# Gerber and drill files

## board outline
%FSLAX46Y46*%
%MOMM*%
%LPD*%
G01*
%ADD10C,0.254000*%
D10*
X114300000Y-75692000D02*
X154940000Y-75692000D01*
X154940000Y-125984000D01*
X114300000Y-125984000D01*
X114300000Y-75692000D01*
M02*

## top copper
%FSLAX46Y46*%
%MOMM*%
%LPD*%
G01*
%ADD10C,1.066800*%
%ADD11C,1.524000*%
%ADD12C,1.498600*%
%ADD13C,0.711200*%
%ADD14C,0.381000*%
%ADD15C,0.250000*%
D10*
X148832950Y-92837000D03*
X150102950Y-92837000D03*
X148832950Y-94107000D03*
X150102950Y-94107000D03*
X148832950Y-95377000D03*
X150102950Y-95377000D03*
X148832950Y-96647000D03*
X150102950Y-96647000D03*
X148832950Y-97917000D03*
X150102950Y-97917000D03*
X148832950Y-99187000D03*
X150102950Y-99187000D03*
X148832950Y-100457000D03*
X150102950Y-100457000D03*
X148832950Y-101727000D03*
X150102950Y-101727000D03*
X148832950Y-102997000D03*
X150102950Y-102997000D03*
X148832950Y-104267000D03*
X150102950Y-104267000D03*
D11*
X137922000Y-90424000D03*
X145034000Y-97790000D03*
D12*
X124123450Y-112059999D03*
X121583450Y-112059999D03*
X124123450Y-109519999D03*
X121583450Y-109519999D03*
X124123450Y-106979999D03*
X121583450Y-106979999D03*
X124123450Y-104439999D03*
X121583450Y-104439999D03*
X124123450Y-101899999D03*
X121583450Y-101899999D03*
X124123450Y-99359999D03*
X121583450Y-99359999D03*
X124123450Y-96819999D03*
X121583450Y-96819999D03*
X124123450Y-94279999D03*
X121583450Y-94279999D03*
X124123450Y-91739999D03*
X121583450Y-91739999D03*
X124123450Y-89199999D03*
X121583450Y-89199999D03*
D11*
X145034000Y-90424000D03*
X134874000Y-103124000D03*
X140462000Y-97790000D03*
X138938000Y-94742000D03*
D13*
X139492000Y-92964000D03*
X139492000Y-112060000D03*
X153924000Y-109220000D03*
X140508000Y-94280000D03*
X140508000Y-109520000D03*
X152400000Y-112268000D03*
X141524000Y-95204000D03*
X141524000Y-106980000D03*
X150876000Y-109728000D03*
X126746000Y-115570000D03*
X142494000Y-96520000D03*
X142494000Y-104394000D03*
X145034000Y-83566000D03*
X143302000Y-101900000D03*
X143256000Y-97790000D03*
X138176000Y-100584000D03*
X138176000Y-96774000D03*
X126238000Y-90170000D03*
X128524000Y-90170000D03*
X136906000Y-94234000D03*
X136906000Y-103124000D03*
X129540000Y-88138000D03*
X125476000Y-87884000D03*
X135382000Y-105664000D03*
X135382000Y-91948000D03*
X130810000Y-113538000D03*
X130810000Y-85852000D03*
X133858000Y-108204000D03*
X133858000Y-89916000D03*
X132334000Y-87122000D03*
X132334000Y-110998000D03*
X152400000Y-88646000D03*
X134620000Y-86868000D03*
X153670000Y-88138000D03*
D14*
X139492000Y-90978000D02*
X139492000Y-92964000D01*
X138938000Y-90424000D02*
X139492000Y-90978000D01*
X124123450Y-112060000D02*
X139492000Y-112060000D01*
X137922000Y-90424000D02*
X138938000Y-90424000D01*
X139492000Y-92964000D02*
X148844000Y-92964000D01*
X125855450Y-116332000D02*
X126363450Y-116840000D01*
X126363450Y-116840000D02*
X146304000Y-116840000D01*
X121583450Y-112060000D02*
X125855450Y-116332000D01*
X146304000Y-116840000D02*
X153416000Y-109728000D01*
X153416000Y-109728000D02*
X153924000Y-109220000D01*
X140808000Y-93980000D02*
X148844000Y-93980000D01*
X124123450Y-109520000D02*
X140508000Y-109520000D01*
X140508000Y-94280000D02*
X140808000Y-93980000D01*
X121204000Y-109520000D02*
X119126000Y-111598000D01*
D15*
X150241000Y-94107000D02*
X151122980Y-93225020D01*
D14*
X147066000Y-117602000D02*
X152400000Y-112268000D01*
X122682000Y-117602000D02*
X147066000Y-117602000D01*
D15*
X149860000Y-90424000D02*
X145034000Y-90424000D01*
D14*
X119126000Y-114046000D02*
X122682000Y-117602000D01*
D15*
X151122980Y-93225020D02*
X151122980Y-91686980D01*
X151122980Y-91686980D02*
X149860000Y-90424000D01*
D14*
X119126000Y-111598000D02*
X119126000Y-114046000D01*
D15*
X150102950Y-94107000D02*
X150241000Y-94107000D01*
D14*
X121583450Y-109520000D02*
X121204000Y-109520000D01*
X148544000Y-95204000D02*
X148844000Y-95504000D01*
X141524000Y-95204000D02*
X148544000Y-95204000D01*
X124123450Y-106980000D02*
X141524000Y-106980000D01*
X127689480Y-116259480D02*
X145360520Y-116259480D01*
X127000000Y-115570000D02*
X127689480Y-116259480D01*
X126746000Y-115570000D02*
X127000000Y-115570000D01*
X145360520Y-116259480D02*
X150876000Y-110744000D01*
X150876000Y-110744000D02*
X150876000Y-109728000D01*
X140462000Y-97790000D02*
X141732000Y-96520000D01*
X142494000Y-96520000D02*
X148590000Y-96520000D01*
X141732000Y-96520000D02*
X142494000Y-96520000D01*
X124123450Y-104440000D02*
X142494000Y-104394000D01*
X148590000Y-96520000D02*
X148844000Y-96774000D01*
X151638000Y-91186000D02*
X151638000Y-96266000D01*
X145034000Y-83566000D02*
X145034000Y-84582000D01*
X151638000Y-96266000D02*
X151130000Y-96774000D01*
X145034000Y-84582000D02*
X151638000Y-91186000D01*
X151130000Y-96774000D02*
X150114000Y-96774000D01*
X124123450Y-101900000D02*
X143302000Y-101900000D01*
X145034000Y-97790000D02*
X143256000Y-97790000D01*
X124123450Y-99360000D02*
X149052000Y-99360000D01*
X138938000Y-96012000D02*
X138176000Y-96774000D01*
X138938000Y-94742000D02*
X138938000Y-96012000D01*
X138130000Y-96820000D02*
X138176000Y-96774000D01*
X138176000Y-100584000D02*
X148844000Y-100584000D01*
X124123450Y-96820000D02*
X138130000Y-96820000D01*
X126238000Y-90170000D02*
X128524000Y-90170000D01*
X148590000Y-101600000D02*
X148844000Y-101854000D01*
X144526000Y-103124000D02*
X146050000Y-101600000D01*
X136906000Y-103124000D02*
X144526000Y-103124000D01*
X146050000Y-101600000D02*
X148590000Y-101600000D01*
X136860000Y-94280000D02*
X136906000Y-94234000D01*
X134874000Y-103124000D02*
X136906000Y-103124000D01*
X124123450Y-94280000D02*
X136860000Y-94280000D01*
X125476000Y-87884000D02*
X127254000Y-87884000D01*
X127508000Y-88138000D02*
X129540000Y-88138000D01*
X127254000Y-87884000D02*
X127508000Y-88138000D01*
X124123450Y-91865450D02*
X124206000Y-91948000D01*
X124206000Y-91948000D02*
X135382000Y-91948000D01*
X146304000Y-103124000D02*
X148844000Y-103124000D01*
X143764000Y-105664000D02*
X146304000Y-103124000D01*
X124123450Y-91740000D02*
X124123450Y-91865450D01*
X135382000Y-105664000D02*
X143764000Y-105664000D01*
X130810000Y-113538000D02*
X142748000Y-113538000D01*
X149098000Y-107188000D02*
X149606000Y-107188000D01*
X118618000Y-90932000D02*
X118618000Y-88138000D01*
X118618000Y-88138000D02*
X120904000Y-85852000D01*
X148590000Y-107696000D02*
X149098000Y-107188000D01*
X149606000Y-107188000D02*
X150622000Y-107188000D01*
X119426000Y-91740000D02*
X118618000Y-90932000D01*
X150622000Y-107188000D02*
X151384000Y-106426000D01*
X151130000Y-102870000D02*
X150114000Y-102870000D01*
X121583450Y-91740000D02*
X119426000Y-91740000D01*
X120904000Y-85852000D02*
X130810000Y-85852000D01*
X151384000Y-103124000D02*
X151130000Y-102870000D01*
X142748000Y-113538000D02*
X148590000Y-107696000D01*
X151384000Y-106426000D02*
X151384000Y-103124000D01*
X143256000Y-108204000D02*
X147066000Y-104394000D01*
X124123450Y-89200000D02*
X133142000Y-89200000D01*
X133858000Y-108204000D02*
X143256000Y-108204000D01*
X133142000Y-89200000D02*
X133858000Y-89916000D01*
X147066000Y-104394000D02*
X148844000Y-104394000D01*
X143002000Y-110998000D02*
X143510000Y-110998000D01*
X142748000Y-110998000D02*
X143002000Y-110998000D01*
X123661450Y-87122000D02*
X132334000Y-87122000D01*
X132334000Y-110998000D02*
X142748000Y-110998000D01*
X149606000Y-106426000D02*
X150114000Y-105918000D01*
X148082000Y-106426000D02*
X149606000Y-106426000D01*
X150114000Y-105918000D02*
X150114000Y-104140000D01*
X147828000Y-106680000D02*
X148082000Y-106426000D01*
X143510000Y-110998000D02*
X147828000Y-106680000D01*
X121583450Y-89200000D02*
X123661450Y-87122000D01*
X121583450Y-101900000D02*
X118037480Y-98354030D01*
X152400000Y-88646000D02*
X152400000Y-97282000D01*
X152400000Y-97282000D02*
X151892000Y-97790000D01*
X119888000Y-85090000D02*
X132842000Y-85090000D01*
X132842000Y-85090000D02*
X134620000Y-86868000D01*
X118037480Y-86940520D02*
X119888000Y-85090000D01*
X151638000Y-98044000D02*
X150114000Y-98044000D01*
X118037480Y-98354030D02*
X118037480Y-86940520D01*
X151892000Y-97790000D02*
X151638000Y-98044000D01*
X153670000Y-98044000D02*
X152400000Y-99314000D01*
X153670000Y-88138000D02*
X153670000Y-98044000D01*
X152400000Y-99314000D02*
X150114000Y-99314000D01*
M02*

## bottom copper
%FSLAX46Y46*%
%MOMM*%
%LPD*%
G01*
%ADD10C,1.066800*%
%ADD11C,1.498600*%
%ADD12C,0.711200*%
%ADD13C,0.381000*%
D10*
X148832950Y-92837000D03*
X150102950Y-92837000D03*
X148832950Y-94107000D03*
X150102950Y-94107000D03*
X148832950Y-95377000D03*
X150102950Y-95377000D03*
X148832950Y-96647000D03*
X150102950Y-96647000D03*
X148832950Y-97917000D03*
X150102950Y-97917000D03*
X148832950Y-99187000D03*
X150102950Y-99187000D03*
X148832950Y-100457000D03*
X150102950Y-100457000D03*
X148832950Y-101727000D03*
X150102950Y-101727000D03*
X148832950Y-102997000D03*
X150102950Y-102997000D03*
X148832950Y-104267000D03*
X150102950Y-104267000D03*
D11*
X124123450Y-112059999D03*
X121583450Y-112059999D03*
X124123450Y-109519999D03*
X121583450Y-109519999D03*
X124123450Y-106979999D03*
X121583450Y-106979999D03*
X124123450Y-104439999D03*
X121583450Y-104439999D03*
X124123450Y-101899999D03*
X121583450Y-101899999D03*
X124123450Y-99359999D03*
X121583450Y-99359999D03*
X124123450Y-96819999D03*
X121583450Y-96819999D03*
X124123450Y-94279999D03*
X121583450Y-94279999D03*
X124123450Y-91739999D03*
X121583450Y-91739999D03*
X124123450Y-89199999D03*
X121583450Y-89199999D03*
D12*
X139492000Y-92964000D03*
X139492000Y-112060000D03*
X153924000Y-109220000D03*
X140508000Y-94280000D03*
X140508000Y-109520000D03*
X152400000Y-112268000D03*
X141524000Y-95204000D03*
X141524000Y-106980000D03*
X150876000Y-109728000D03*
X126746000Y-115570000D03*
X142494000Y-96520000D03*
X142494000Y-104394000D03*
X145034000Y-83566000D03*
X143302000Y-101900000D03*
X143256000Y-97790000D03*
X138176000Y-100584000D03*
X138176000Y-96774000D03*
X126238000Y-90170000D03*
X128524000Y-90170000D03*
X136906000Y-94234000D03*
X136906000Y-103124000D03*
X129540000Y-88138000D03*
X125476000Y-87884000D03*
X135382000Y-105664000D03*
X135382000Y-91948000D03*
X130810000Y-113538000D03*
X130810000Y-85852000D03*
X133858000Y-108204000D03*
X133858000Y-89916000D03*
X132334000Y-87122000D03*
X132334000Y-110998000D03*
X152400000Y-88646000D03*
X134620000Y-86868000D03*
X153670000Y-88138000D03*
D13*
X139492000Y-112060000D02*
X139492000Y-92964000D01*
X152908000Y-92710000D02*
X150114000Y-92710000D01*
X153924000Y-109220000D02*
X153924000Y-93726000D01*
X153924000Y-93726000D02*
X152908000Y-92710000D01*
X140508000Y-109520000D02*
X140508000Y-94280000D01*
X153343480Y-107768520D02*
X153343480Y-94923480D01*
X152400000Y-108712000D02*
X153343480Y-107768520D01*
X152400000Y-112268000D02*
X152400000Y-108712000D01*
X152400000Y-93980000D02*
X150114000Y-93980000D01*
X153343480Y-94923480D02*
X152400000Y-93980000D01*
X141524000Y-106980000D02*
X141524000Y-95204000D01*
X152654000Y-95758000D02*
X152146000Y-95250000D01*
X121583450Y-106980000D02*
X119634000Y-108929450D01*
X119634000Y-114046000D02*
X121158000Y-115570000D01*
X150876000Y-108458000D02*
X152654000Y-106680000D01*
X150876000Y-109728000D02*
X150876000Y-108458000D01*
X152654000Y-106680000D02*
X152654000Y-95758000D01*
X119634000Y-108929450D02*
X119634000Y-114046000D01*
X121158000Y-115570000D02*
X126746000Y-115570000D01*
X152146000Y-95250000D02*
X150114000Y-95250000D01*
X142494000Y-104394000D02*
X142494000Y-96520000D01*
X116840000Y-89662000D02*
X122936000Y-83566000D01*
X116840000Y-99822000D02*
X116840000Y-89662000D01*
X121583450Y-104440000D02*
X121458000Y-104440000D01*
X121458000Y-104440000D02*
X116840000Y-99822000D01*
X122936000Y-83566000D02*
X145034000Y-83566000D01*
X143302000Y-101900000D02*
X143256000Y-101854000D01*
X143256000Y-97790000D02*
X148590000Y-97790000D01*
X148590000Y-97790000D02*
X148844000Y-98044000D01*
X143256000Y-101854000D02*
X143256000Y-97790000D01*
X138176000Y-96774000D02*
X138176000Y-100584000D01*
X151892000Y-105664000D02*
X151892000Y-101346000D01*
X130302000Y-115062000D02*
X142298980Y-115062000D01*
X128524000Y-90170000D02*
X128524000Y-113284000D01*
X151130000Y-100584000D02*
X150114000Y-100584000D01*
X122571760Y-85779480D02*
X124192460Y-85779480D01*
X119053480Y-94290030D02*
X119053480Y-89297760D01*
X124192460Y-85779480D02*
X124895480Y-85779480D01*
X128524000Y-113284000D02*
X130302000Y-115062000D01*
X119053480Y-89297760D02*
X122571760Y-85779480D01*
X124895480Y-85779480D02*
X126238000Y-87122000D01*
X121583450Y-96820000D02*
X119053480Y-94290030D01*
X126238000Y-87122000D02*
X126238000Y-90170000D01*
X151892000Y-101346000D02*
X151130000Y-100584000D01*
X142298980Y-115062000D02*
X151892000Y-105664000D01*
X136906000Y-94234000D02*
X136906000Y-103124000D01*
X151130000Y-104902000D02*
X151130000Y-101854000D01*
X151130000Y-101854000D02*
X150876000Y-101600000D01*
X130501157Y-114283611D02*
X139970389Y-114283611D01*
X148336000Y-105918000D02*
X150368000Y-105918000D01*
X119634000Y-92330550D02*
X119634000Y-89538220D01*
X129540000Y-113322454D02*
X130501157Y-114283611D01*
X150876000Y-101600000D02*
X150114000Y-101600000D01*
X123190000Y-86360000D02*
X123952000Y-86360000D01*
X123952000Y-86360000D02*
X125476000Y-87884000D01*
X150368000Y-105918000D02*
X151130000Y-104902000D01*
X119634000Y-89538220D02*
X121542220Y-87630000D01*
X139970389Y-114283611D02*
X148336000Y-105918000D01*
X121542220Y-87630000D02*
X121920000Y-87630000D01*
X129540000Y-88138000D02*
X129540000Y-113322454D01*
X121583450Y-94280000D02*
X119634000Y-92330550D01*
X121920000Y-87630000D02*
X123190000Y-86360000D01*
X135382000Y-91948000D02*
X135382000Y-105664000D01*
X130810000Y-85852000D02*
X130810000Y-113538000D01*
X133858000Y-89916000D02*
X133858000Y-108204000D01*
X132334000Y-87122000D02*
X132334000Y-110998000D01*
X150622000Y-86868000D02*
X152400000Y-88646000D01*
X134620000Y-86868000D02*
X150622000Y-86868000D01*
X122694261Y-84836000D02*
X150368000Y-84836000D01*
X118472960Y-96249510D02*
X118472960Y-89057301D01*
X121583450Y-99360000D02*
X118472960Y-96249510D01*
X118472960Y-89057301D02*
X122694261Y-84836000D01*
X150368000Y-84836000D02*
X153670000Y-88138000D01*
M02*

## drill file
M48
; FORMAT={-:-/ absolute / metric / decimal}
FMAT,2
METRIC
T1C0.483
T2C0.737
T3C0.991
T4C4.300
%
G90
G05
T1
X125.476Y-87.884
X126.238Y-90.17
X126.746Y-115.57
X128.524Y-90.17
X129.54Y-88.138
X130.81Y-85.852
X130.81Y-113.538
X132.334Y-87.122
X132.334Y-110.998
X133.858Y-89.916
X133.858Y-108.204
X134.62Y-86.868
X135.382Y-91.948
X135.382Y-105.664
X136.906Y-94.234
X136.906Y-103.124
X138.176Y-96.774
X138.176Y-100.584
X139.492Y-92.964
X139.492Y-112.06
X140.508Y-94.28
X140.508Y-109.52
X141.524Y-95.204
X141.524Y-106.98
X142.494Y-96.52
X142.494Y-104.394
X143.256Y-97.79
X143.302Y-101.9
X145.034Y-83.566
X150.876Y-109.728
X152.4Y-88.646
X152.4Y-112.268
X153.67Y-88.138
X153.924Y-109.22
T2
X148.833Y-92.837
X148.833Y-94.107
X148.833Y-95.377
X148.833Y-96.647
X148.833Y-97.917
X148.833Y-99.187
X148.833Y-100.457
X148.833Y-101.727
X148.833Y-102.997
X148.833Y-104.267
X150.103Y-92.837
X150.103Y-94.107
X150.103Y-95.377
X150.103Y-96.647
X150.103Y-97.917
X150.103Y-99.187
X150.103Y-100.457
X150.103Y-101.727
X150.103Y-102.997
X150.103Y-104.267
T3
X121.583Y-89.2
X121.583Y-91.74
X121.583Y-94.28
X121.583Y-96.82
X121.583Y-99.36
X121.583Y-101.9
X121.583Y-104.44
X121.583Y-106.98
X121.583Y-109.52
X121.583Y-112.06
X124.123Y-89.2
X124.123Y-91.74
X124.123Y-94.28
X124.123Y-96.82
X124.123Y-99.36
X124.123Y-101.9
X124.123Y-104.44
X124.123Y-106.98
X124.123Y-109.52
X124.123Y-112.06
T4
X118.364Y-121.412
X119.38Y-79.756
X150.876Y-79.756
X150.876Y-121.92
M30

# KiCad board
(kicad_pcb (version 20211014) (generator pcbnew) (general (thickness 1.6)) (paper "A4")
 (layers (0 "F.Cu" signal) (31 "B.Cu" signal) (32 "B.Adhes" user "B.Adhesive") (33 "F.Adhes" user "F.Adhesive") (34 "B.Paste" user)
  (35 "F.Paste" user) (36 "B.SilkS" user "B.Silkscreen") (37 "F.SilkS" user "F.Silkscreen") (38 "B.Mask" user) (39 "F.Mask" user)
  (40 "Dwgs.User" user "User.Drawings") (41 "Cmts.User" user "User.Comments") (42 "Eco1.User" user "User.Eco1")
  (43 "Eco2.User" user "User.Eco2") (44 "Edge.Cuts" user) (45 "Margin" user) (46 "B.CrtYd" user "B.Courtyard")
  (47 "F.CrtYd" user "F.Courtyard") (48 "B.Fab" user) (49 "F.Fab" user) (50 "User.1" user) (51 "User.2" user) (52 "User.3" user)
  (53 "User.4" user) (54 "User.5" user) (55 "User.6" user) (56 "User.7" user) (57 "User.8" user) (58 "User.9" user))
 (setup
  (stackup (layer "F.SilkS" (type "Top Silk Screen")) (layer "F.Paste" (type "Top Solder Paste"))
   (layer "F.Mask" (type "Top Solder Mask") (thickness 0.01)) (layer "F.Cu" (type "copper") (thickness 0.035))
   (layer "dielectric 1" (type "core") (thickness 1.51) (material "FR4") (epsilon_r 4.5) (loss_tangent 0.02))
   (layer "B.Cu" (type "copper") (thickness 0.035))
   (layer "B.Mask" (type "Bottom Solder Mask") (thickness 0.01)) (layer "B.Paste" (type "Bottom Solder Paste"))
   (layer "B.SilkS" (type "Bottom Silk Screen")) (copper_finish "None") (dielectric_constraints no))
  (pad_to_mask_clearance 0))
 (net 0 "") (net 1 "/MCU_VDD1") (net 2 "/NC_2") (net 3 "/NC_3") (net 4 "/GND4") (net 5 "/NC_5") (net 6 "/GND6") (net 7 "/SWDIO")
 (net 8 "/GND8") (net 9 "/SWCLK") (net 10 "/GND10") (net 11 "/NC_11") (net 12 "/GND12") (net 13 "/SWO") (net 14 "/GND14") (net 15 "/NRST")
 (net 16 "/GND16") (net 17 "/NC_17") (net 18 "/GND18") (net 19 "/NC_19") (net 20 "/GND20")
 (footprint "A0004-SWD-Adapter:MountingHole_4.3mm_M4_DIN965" (layer "F.Cu") (at 150.876 79.756)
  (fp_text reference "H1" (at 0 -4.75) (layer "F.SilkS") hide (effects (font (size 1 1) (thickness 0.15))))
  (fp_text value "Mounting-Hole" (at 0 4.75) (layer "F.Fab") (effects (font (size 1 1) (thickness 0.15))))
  (pad "" np_thru_hole circle (at 0 0) (size 4.3 4.3) (drill 4.3) (layers *.Cu *.Mask)))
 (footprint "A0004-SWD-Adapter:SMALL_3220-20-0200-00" (layer "F.Cu") (at 150.10295 98.552 -90)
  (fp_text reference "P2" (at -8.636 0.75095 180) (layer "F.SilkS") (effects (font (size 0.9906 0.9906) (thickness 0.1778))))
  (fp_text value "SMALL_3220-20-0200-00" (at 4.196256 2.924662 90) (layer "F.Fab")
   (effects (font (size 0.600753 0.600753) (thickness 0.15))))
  (pad "1" thru_hole circle (at -5.715 1.27 270) (size 1.0668 1.0668) (drill 0.7366) (layers *.Cu *.Mask) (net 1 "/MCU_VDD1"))
  (pad "2" thru_hole circle (at -5.715 0 270) (size 1.0668 1.0668) (drill 0.7366) (layers *.Cu *.Mask) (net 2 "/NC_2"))
  (pad "3" thru_hole circle (at -4.445 1.27 270) (size 1.0668 1.0668) (drill 0.7366) (layers *.Cu *.Mask) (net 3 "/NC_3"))
  (pad "4" thru_hole circle (at -4.445 0 270) (size 1.0668 1.0668) (drill 0.7366) (layers *.Cu *.Mask) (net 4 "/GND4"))
  (pad "5" thru_hole circle (at -3.175 1.27 270) (size 1.0668 1.0668) (drill 0.7366) (layers *.Cu *.Mask) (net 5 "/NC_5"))
  (pad "6" thru_hole circle (at -3.175 0 270) (size 1.0668 1.0668) (drill 0.7366) (layers *.Cu *.Mask) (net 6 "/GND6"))
  (pad "7" thru_hole circle (at -1.905 1.27 270) (size 1.0668 1.0668) (drill 0.7366) (layers *.Cu *.Mask) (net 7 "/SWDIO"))
  (pad "8" thru_hole circle (at -1.905 0 270) (size 1.0668 1.0668) (drill 0.7366) (layers *.Cu *.Mask) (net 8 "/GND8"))
  (pad "9" thru_hole circle (at -0.635 1.27 270) (size 1.0668 1.0668) (drill 0.7366) (layers *.Cu *.Mask) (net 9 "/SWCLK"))
  (pad "10" thru_hole circle (at -0.635 0 270) (size 1.0668 1.0668) (drill 0.7366) (layers *.Cu *.Mask) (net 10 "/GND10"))
  (pad "11" thru_hole circle (at 0.635 1.27 270) (size 1.0668 1.0668) (drill 0.7366) (layers *.Cu *.Mask) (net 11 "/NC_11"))
  (pad "12" thru_hole circle (at 0.635 0 270) (size 1.0668 1.0668) (drill 0.7366) (layers *.Cu *.Mask) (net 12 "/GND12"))
  (pad "13" thru_hole circle (at 1.905 1.27 270) (size 1.0668 1.0668) (drill 0.7366) (layers *.Cu *.Mask) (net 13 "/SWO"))
  (pad "14" thru_hole circle (at 1.905 0 270) (size 1.0668 1.0668) (drill 0.7366) (layers *.Cu *.Mask) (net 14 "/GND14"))
  (pad "15" thru_hole circle (at 3.175 1.27 270) (size 1.0668 1.0668) (drill 0.7366) (layers *.Cu *.Mask) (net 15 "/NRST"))
  (pad "16" thru_hole circle (at 3.175 0 270) (size 1.0668 1.0668) (drill 0.7366) (layers *.Cu *.Mask) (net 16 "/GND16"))
  (pad "17" thru_hole circle (at 4.445 1.27 270) (size 1.0668 1.0668) (drill 0.7366) (layers *.Cu *.Mask) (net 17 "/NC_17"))
  (pad "18" thru_hole circle (at 4.445 0 270) (size 1.0668 1.0668) (drill 0.7366) (layers *.Cu *.Mask) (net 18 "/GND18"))
  (pad "19" thru_hole circle (at 5.715 1.27 270) (size 1.0668 1.0668) (drill 0.7366) (layers *.Cu *.Mask) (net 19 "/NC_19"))
  (pad "20" thru_hole circle (at 5.715 0 270) (size 1.0668 1.0668) (drill 0.7366) (layers *.Cu *.Mask) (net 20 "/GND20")))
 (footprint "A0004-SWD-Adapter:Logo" (layer "F.Cu") (at 135.382 119.888)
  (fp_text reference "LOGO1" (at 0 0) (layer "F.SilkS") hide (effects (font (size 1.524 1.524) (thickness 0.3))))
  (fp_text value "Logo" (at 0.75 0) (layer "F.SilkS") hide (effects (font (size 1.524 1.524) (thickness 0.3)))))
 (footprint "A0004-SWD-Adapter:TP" (layer "F.Cu") (at 137.922 90.424)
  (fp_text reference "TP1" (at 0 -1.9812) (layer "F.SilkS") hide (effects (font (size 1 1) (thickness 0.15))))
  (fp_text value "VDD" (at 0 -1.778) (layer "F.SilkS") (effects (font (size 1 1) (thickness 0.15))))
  (pad "1" smd circle (at 0 0) (size 1.524 1.524) (layers "F.Cu" "F.Paste" "F.Mask") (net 1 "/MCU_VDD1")))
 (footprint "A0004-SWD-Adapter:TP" (layer "F.Cu") (at 145.034 97.79)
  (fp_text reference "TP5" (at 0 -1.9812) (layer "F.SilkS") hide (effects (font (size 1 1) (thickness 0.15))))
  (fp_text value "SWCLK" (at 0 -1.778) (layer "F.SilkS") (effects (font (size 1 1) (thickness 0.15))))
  (pad "1" smd circle (at 0 0) (size 1.524 1.524) (layers "F.Cu" "F.Paste" "F.Mask") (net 9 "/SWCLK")))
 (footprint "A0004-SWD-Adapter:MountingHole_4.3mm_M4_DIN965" (layer "F.Cu") (at 118.364 121.412)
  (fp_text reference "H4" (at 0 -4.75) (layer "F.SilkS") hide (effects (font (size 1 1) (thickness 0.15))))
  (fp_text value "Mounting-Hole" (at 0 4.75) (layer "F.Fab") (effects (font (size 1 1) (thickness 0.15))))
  (pad "" np_thru_hole circle (at 0 0) (size 4.3 4.3) (drill 4.3) (layers *.Cu *.Mask)))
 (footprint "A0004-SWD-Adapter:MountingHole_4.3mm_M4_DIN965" (layer "F.Cu") (at 119.38 79.756)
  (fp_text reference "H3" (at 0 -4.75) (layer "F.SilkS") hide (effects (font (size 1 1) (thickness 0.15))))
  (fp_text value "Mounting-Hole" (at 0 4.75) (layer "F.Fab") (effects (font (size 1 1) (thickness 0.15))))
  (pad "" np_thru_hole circle (at 0 0) (size 4.3 4.3) (drill 4.3) (layers *.Cu *.Mask)))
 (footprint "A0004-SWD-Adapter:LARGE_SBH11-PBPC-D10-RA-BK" (layer "F.Cu") (at 121.58345 112.059999 90)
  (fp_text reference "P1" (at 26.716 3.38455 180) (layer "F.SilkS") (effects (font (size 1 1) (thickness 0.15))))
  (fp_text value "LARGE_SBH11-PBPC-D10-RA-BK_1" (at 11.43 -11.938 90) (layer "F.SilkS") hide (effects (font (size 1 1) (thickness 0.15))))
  (pad "1" thru_hole circle (at 0 2.54 90) (size 1.4986 1.4986) (drill 0.9906) (layers *.Cu *.Mask) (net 1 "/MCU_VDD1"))
  (pad "2" thru_hole circle (at 0 0 90) (size 1.4986 1.4986) (drill 0.9906) (layers *.Cu *.Mask) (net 2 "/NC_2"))
  (pad "3" thru_hole circle (at 2.54 2.54 90) (size 1.4986 1.4986) (drill 0.9906) (layers *.Cu *.Mask) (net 3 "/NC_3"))
  (pad "4" thru_hole circle (at 2.54 0 90) (size 1.4986 1.4986) (drill 0.9906) (layers *.Cu *.Mask) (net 4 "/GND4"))
  (pad "5" thru_hole circle (at 5.08 2.54 90) (size 1.4986 1.4986) (drill 0.9906) (layers *.Cu *.Mask) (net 5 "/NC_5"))
  (pad "6" thru_hole circle (at 5.08 0 90) (size 1.4986 1.4986) (drill 0.9906) (layers *.Cu *.Mask) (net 6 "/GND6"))
  (pad "7" thru_hole circle (at 7.62 2.54 90) (size 1.4986 1.4986) (drill 0.9906) (layers *.Cu *.Mask) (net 7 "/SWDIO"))
  (pad "8" thru_hole circle (at 7.62 0 90) (size 1.4986 1.4986) (drill 0.9906) (layers *.Cu *.Mask) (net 8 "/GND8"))
  (pad "9" thru_hole circle (at 10.16 2.54 90) (size 1.4986 1.4986) (drill 0.9906) (layers *.Cu *.Mask) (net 9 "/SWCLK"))
  (pad "10" thru_hole circle (at 10.16 0 90) (size 1.4986 1.4986) (drill 0.9906) (layers *.Cu *.Mask) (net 10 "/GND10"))
  (pad "11" thru_hole circle (at 12.7 2.54 90) (size 1.4986 1.4986) (drill 0.9906) (layers *.Cu *.Mask) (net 11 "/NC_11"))
  (pad "12" thru_hole circle (at 12.7 0 90) (size 1.4986 1.4986) (drill 0.9906) (layers *.Cu *.Mask) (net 12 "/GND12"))
  (pad "13" thru_hole circle (at 15.24 2.54 90) (size 1.4986 1.4986) (drill 0.9906) (layers *.Cu *.Mask) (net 13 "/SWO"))
  (pad "14" thru_hole circle (at 15.24 0 90) (size 1.4986 1.4986) (drill 0.9906) (layers *.Cu *.Mask) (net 14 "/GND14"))
  (pad "15" thru_hole circle (at 17.78 2.54 90) (size 1.4986 1.4986) (drill 0.9906) (layers *.Cu *.Mask) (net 15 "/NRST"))
  (pad "16" thru_hole circle (at 17.78 0 90) (size 1.4986 1.4986) (drill 0.9906) (layers *.Cu *.Mask) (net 16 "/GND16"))
  (pad "17" thru_hole circle (at 20.32 2.54 90) (size 1.4986 1.4986) (drill 0.9906) (layers *.Cu *.Mask) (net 17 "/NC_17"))
  (pad "18" thru_hole circle (at 20.32 0 90) (size 1.4986 1.4986) (drill 0.9906) (layers *.Cu *.Mask) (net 18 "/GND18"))
  (pad "19" thru_hole circle (at 22.86 2.54 90) (size 1.4986 1.4986) (drill 0.9906) (layers *.Cu *.Mask) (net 19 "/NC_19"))
  (pad "20" thru_hole circle (at 22.86 0 90) (size 1.4986 1.4986) (drill 0.9906) (layers *.Cu *.Mask) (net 20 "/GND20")))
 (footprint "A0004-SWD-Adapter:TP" (layer "F.Cu") (at 145.034 90.424)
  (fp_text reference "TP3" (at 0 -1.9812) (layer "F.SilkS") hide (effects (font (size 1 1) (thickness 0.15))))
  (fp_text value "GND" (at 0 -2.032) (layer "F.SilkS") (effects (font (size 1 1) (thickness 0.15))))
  (pad "1" smd circle (at 0 0) (size 1.524 1.524) (layers "F.Cu" "F.Paste" "F.Mask") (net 4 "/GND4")))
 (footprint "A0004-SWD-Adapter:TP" (layer "F.Cu") (at 134.874 103.124)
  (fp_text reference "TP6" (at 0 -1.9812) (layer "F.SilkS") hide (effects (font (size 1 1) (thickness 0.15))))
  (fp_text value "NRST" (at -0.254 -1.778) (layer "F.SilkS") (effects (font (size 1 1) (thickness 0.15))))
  (pad "1" smd circle (at 0 0) (size 1.524 1.524) (layers "F.Cu" "F.Paste" "F.Mask") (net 15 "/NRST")))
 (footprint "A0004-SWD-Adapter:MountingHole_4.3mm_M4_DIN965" (layer "F.Cu") (at 150.876 121.92)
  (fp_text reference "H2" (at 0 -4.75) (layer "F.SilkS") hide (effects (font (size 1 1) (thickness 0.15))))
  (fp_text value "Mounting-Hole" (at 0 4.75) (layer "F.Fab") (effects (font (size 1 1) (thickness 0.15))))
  (pad "" np_thru_hole circle (at 0 0) (size 4.3 4.3) (drill 4.3) (layers *.Cu *.Mask)))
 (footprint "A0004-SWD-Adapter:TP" (layer "F.Cu") (at 140.462 97.79)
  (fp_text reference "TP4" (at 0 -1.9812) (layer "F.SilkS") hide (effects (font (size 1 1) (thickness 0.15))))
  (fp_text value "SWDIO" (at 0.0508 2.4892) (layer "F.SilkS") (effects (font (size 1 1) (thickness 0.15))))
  (pad "1" smd circle (at 0 0) (size 1.524 1.524) (layers "F.Cu" "F.Paste" "F.Mask") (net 7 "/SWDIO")))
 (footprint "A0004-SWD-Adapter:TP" (layer "F.Cu") (at 138.938 94.742)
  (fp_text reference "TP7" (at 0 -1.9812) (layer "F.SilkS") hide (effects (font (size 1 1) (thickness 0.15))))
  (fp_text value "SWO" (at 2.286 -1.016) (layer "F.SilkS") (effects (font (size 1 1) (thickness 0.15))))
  (pad "1" smd circle (at 0 0) (size 1.524 1.524) (layers "F.Cu" "F.Paste" "F.Mask") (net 13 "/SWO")))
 (gr_rect (start 114.3 75.692) (end 154.94 125.984) (layer "Edge.Cuts") (width 0.254) (fill none))
 (segment (start 139.492 90.978) (end 139.492 92.964) (width 0.381) (layer "F.Cu") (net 1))
 (segment (start 138.938 90.424) (end 139.492 90.978) (width 0.381) (layer "F.Cu") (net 1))
 (segment (start 124.12345 112.06) (end 139.492 112.06) (width 0.381) (layer "F.Cu") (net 1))
 (segment (start 137.922 90.424) (end 138.938 90.424) (width 0.381) (layer "F.Cu") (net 1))
 (segment (start 139.492 92.964) (end 148.844 92.964) (width 0.381) (layer "F.Cu") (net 1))
 (via (at 139.492 92.964) (size 0.7112) (drill 0.4826) (layers "F.Cu" "B.Cu") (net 1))
 (via (at 139.492 112.06) (size 0.7112) (drill 0.4826) (layers "F.Cu" "B.Cu") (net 1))
 (segment (start 139.492 112.06) (end 139.492 92.964) (width 0.381) (layer "B.Cu") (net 1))
 (segment (start 125.85545 116.332) (end 126.36345 116.84) (width 0.381) (layer "F.Cu") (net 2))
 (segment (start 126.36345 116.84) (end 146.304 116.84) (width 0.381) (layer "F.Cu") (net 2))
 (segment (start 121.58345 112.06) (end 125.85545 116.332) (width 0.381) (layer "F.Cu") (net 2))
 (segment (start 146.304 116.84) (end 153.416 109.728) (width 0.381) (layer "F.Cu") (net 2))
 (segment (start 153.416 109.728) (end 153.924 109.22) (width 0.381) (layer "F.Cu") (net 2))
 (via (at 153.924 109.22) (size 0.7112) (drill 0.4826) (layers "F.Cu" "B.Cu") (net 2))
 (segment (start 152.908 92.71) (end 150.114 92.71) (width 0.381) (layer "B.Cu") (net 2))
 (segment (start 153.924 109.22) (end 153.924 93.726) (width 0.381) (layer "B.Cu") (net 2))
 (segment (start 153.924 93.726) (end 152.908 92.71) (width 0.381) (layer "B.Cu") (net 2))
 (segment (start 140.808 93.98) (end 148.844 93.98) (width 0.381) (layer "F.Cu") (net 3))
 (segment (start 124.12345 109.52) (end 140.508 109.52) (width 0.381) (layer "F.Cu") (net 3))
 (segment (start 140.508 94.28) (end 140.808 93.98) (width 0.381) (layer "F.Cu") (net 3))
 (via (at 140.508 94.28) (size 0.7112) (drill 0.4826) (layers "F.Cu" "B.Cu") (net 3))
 (via (at 140.508 109.52) (size 0.7112) (drill 0.4826) (layers "F.Cu" "B.Cu") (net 3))
 (segment (start 140.508 109.52) (end 140.508 94.28) (width 0.381) (layer "B.Cu") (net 3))
 (segment (start 121.204 109.52) (end 119.126 111.598) (width 0.381) (layer "F.Cu") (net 4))
 (segment (start 150.241 94.107) (end 151.12298 93.22502) (width 0.25) (layer "F.Cu") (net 4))
 (segment (start 147.066 117.602) (end 152.4 112.268) (width 0.381) (layer "F.Cu") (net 4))
 (segment (start 122.682 117.602) (end 147.066 117.602) (width 0.381) (layer "F.Cu") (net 4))
 (segment (start 149.86 90.424) (end 145.034 90.424) (width 0.25) (layer "F.Cu") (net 4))
 (segment (start 119.126 114.046) (end 122.682 117.602) (width 0.381) (layer "F.Cu") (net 4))
 (segment (start 151.12298 93.22502) (end 151.12298 91.68698) (width 0.25) (layer "F.Cu") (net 4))
 (segment (start 151.12298 91.68698) (end 149.86 90.424) (width 0.25) (layer "F.Cu") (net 4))
 (segment (start 119.126 111.598) (end 119.126 114.046) (width 0.381) (layer "F.Cu") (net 4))
 (segment (start 150.10295 94.107) (end 150.241 94.107) (width 0.25) (layer "F.Cu") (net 4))
 (segment (start 121.58345 109.52) (end 121.204 109.52) (width 0.381) (layer "F.Cu") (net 4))
 (via (at 152.4 112.268) (size 0.7112) (drill 0.4826) (layers "F.Cu" "B.Cu") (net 4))
 (segment (start 153.34348 107.76852) (end 153.34348 94.92348) (width 0.381) (layer "B.Cu") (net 4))
 (segment (start 152.4 108.712) (end 153.34348 107.76852) (width 0.381) (layer "B.Cu") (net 4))
 (segment (start 152.4 112.268) (end 152.4 108.712) (width 0.381) (layer "B.Cu") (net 4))
 (segment (start 152.4 93.98) (end 150.114 93.98) (width 0.381) (layer "B.Cu") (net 4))
 (segment (start 153.34348 94.92348) (end 152.4 93.98) (width 0.381) (layer "B.Cu") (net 4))
 (segment (start 148.544 95.204) (end 148.844 95.504) (width 0.381) (layer "F.Cu") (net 5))
 (segment (start 141.524 95.204) (end 148.544 95.204) (width 0.381) (layer "F.Cu") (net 5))
 (segment (start 124.12345 106.98) (end 141.524 106.98) (width 0.381) (layer "F.Cu") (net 5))
 (via (at 141.524 95.204) (size 0.7112) (drill 0.4826) (layers "F.Cu" "B.Cu") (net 5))
 (via (at 141.524 106.98) (size 0.7112) (drill 0.4826) (layers "F.Cu" "B.Cu") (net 5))
 (segment (start 141.524 106.98) (end 141.524 95.204) (width 0.381) (layer "B.Cu") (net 5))
 (segment (start 127.68948 116.25948) (end 145.36052 116.25948) (width 0.381) (layer "F.Cu") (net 6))
 (segment (start 127 115.57) (end 127.68948 116.25948) (width 0.381) (layer "F.Cu") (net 6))
 (segment (start 126.746 115.57) (end 127 115.57) (width 0.381) (layer "F.Cu") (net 6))
 (segment (start 145.36052 116.25948) (end 150.876 110.744) (width 0.381) (layer "F.Cu") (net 6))
 (segment (start 150.876 110.744) (end 150.876 109.728) (width 0.381) (layer "F.Cu") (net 6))
 (via (at 150.876 109.728) (size 0.7112) (drill 0.4826) (layers "F.Cu" "B.Cu") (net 6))
 (via (at 126.746 115.57) (size 0.7112) (drill 0.4826) (layers "F.Cu" "B.Cu") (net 6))
 (segment (start 152.654 95.758) (end 152.146 95.25) (width 0.381) (layer "B.Cu") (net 6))
 (segment (start 121.58345 106.98) (end 119.634 108.92945) (width 0.381) (layer "B.Cu") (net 6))
 (segment (start 119.634 114.046) (end 121.158 115.57) (width 0.381) (layer "B.Cu") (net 6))
 (segment (start 150.876 108.458) (end 152.654 106.68) (width 0.381) (layer "B.Cu") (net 6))
 (segment (start 150.876 109.728) (end 150.876 108.458) (width 0.381) (layer "B.Cu") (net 6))
 (segment (start 152.654 106.68) (end 152.654 95.758) (width 0.381) (layer "B.Cu") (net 6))
 (segment (start 119.634 108.92945) (end 119.634 114.046) (width 0.381) (layer "B.Cu") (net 6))
 (segment (start 121.158 115.57) (end 126.746 115.57) (width 0.381) (layer "B.Cu") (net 6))
 (segment (start 152.146 95.25) (end 150.114 95.25) (width 0.381) (layer "B.Cu") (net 6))
 (segment (start 140.462 97.79) (end 141.732 96.52) (width 0.381) (layer "F.Cu") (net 7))
 (segment (start 142.494 96.52) (end 148.59 96.52) (width 0.381) (layer "F.Cu") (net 7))
 (segment (start 141.732 96.52) (end 142.494 96.52) (width 0.381) (layer "F.Cu") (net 7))
 (segment (start 124.12345 104.44) (end 142.494 104.394) (width 0.381) (layer "F.Cu") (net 7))
 (segment (start 148.59 96.52) (end 148.844 96.774) (width 0.381) (layer "F.Cu") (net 7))
 (via (at 142.494 96.52) (size 0.7112) (drill 0.4826) (layers "F.Cu" "B.Cu") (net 7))
 (via (at 142.494 104.394) (size 0.7112) (drill 0.4826) (layers "F.Cu" "B.Cu") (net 7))
 (segment (start 142.494 104.394) (end 142.494 96.52) (width 0.381) (layer "B.Cu") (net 7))
 (segment (start 151.638 91.186) (end 151.638 96.266) (width 0.381) (layer "F.Cu") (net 8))
 (segment (start 145.034 83.566) (end 145.034 84.582) (width 0.381) (layer "F.Cu") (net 8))
 (segment (start 151.638 96.266) (end 151.13 96.774) (width 0.381) (layer "F.Cu") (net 8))
 (segment (start 145.034 84.582) (end 151.638 91.186) (width 0.381) (layer "F.Cu") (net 8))
 (segment (start 151.13 96.774) (end 150.114 96.774) (width 0.381) (layer "F.Cu") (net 8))
 (via (at 145.034 83.566) (size 0.7112) (drill 0.4826) (layers "F.Cu" "B.Cu") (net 8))
 (segment (start 116.84 89.662) (end 122.936 83.566) (width 0.381) (layer "B.Cu") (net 8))
 (segment (start 116.84 99.822) (end 116.84 89.662) (width 0.381) (layer "B.Cu") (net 8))
 (segment (start 121.58345 104.44) (end 121.458 104.44) (width 0.381) (layer "B.Cu") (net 8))
 (segment (start 121.458 104.44) (end 116.84 99.822) (width 0.381) (layer "B.Cu") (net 8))
 (segment (start 122.936 83.566) (end 145.034 83.566) (width 0.381) (layer "B.Cu") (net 8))
 (segment (start 124.12345 101.9) (end 143.302 101.9) (width 0.381) (layer "F.Cu") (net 9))
 (segment (start 145.034 97.79) (end 143.256 97.79) (width 0.381) (layer "F.Cu") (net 9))
 (via (at 143.302 101.9) (size 0.7112) (drill 0.4826) (layers "F.Cu" "B.Cu") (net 9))
 (via (at 143.256 97.79) (size 0.7112) (drill 0.4826) (layers "F.Cu" "B.Cu") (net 9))
 (segment (start 143.302 101.9) (end 143.256 101.854) (width 0.381) (layer "B.Cu") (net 9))
 (segment (start 143.256 97.79) (end 148.59 97.79) (width 0.381) (layer "B.Cu") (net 9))
 (segment (start 148.59 97.79) (end 148.844 98.044) (width 0.381) (layer "B.Cu") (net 9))
 (segment (start 143.256 101.854) (end 143.256 97.79) (width 0.381) (layer "B.Cu") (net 9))
 (segment (start 124.12345 99.36) (end 149.052 99.36) (width 0.381) (layer "F.Cu") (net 11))
 (segment (start 138.938 96.012) (end 138.176 96.774) (width 0.381) (layer "F.Cu") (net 13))
 (segment (start 138.938 94.742) (end 138.938 96.012) (width 0.381) (layer "F.Cu") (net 13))
 (segment (start 138.13 96.82) (end 138.176 96.774) (width 0.381) (layer "F.Cu") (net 13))
 (segment (start 138.176 100.584) (end 148.844 100.584) (width 0.381) (layer "F.Cu") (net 13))
 (segment (start 124.12345 96.82) (end 138.13 96.82) (width 0.381) (layer "F.Cu") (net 13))
 (via (at 138.176 100.584) (size 0.7112) (drill 0.4826) (layers "F.Cu" "B.Cu") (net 13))
 (via (at 138.176 96.774) (size 0.7112) (drill 0.4826) (layers "F.Cu" "B.Cu") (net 13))
 (segment (start 138.176 96.774) (end 138.176 100.584) (width 0.381) (layer "B.Cu") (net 13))
 (segment (start 126.238 90.17) (end 128.524 90.17) (width 0.381) (layer "F.Cu") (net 14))
 (via (at 126.238 90.17) (size 0.7112) (drill 0.4826) (layers "F.Cu" "B.Cu") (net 14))
 (via (at 128.524 90.17) (size 0.7112) (drill 0.4826) (layers "F.Cu" "B.Cu") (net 14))
 (segment (start 151.892 105.664) (end 151.892 101.346) (width 0.381) (layer "B.Cu") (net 14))
 (segment (start 130.302 115.062) (end 142.29898 115.062) (width 0.381) (layer "B.Cu") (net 14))
 (segment (start 128.524 90.17) (end 128.524 113.284) (width 0.381) (layer "B.Cu") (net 14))
 (segment (start 151.13 100.584) (end 150.114 100.584) (width 0.381) (layer "B.Cu") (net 14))
 (segment (start 122.57176 85.77948) (end 124.19246 85.77948) (width 0.381) (layer "B.Cu") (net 14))
 (segment (start 119.05348 94.29003) (end 119.05348 89.29776) (width 0.381) (layer "B.Cu") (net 14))
 (segment (start 124.19246 85.77948) (end 124.89548 85.77948) (width 0.381) (layer "B.Cu") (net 14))
 (segment (start 128.524 113.284) (end 130.302 115.062) (width 0.381) (layer "B.Cu") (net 14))
 (segment (start 119.05348 89.29776) (end 122.57176 85.77948) (width 0.381) (layer "B.Cu") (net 14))
 (segment (start 124.89548 85.77948) (end 126.238 87.122) (width 0.381) (layer "B.Cu") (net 14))
 (segment (start 121.58345 96.82) (end 119.05348 94.29003) (width 0.381) (layer "B.Cu") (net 14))
 (segment (start 126.238 87.122) (end 126.238 90.17) (width 0.381) (layer "B.Cu") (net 14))
 (segment (start 151.892 101.346) (end 151.13 100.584) (width 0.381) (layer "B.Cu") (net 14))
 (segment (start 142.29898 115.062) (end 151.892 105.664) (width 0.381) (layer "B.Cu") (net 14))
 (segment (start 148.59 101.6) (end 148.844 101.854) (width 0.381) (layer "F.Cu") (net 15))
 (segment (start 144.526 103.124) (end 146.05 101.6) (width 0.381) (layer "F.Cu") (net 15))
 (segment (start 136.906 103.124) (end 144.526 103.124) (width 0.381) (layer "F.Cu") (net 15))
 (segment (start 146.05 101.6) (end 148.59 101.6) (width 0.381) (layer "F.Cu") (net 15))
 (segment (start 136.86 94.28) (end 136.906 94.234) (width 0.381) (layer "F.Cu") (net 15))
 (segment (start 134.874 103.124) (end 136.906 103.124) (width 0.381) (layer "F.Cu") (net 15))
 (segment (start 124.12345 94.28) (end 136.86 94.28) (width 0.381) (layer "F.Cu") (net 15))
 (via (at 136.906 94.234) (size 0.7112) (drill 0.4826) (layers "F.Cu" "B.Cu") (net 15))
 (via (at 136.906 103.124) (size 0.7112) (drill 0.4826) (layers "F.Cu" "B.Cu") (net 15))
 (segment (start 136.906 94.234) (end 136.906 103.124) (width 0.381) (layer "B.Cu") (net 15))
 (segment (start 125.476 87.884) (end 127.254 87.884) (width 0.381) (layer "F.Cu") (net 16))
 (segment (start 127.508 88.138) (end 129.54 88.138) (width 0.381) (layer "F.Cu") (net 16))
 (segment (start 127.254 87.884) (end 127.508 88.138) (width 0.381) (layer "F.Cu") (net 16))
 (via (at 129.54 88.138) (size 0.7112) (drill 0.4826) (layers "F.Cu" "B.Cu") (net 16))
 (via (at 125.476 87.884) (size 0.7112) (drill 0.4826) (layers "F.Cu" "B.Cu") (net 16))
 (segment (start 151.13 104.902) (end 151.13 101.854) (width 0.381) (layer "B.Cu") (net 16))
 (segment (start 151.13 101.854) (end 150.876 101.6) (width 0.381) (layer "B.Cu") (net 16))
 (segment (start 130.501157 114.283611) (end 139.970389 114.283611) (width 0.381) (layer "B.Cu") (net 16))
 (segment (start 148.336 105.918) (end 150.368 105.918) (width 0.381) (layer "B.Cu") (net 16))
 (segment (start 119.634 92.33055) (end 119.634 89.53822) (width 0.381) (layer "B.Cu") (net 16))
 (segment (start 129.54 113.322454) (end 130.501157 114.283611) (width 0.381) (layer "B.Cu") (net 16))
 (segment (start 150.876 101.6) (end 150.114 101.6) (width 0.381) (layer "B.Cu") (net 16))
 (segment (start 123.19 86.36) (end 123.952 86.36) (width 0.381) (layer "B.Cu") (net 16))
 (segment (start 123.952 86.36) (end 125.476 87.884) (width 0.381) (layer "B.Cu") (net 16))
 (segment (start 150.368 105.918) (end 151.13 104.902) (width 0.381) (layer "B.Cu") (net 16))
 (segment (start 119.634 89.53822) (end 121.54222 87.63) (width 0.381) (layer "B.Cu") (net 16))
 (segment (start 139.970389 114.283611) (end 148.336 105.918) (width 0.381) (layer "B.Cu") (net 16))
 (segment (start 121.54222 87.63) (end 121.92 87.63) (width 0.381) (layer "B.Cu") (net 16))
 (segment (start 129.54 88.138) (end 129.54 113.322454) (width 0.381) (layer "B.Cu") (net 16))
 (segment (start 121.58345 94.28) (end 119.634 92.33055) (width 0.381) (layer "B.Cu") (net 16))
 (segment (start 121.92 87.63) (end 123.19 86.36) (width 0.381) (layer "B.Cu") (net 16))
 (segment (start 124.12345 91.86545) (end 124.206 91.948) (width 0.381) (layer "F.Cu") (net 17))
 (segment (start 124.206 91.948) (end 135.382 91.948) (width 0.381) (layer "F.Cu") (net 17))
 (segment (start 146.304 103.124) (end 148.844 103.124) (width 0.381) (layer "F.Cu") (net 17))
 (segment (start 143.764 105.664) (end 146.304 103.124) (width 0.381) (layer "F.Cu") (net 17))
 (segment (start 124.12345 91.74) (end 124.12345 91.86545) (width 0.381) (layer "F.Cu") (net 17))
 (segment (start 135.382 105.664) (end 143.764 105.664) (width 0.381) (layer "F.Cu") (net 17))
 (via (at 135.382 105.664) (size 0.7112) (drill 0.4826) (layers "F.Cu" "B.Cu") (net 17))
 (via (at 135.382 91.948) (size 0.7112) (drill 0.4826) (layers "F.Cu" "B.Cu") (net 17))
 (segment (start 135.382 91.948) (end 135.382 105.664) (width 0.381) (layer "B.Cu") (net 17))
 (segment (start 130.81 113.538) (end 142.748 113.538) (width 0.381) (layer "F.Cu") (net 18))
 (segment (start 149.098 107.188) (end 149.606 107.188) (width 0.381) (layer "F.Cu") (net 18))
 (segment (start 118.618 90.932) (end 118.618 88.138) (width 0.381) (layer "F.Cu") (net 18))
 (segment (start 118.618 88.138) (end 120.904 85.852) (width 0.381) (layer "F.Cu") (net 18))
 (segment (start 148.59 107.696) (end 149.098 107.188) (width 0.381) (layer "F.Cu") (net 18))
 (segment (start 149.606 107.188) (end 150.622 107.188) (width 0.381) (layer "F.Cu") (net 18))
 (segment (start 119.426 91.74) (end 118.618 90.932) (width 0.381) (layer "F.Cu") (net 18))
 (segment (start 150.622 107.188) (end 151.384 106.426) (width 0.381) (layer "F.Cu") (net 18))
 (segment (start 151.13 102.87) (end 150.114 102.87) (width 0.381) (layer "F.Cu") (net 18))
 (segment (start 121.58345 91.74) (end 119.426 91.74) (width 0.381) (layer "F.Cu") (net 18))
 (segment (start 120.904 85.852) (end 130.81 85.852) (width 0.381) (layer "F.Cu") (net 18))
 (segment (start 151.384 103.124) (end 151.13 102.87) (width 0.381) (layer "F.Cu") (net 18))
 (segment (start 142.748 113.538) (end 148.59 107.696) (width 0.381) (layer "F.Cu") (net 18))
 (segment (start 151.384 106.426) (end 151.384 103.124) (width 0.381) (layer "F.Cu") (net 18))
 (via (at 130.81 113.538) (size 0.7112) (drill 0.4826) (layers "F.Cu" "B.Cu") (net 18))
 (via (at 130.81 85.852) (size 0.7112) (drill 0.4826) (layers "F.Cu" "B.Cu") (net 18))
 (segment (start 130.81 85.852) (end 130.81 113.538) (width 0.381) (layer "B.Cu") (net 18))
 (segment (start 143.256 108.204) (end 147.066 104.394) (width 0.381) (layer "F.Cu") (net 19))
 (segment (start 124.12345 89.2) (end 133.142 89.2) (width 0.381) (layer "F.Cu") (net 19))
 (segment (start 133.858 108.204) (end 143.256 108.204) (width 0.381) (layer "F.Cu") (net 19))
 (segment (start 133.142 89.2) (end 133.858 89.916) (width 0.381) (layer "F.Cu") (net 19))
 (segment (start 147.066 104.394) (end 148.844 104.394) (width 0.381) (layer "F.Cu") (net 19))
 (via (at 133.858 108.204) (size 0.7112) (drill 0.4826) (layers "F.Cu" "B.Cu") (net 19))
 (via (at 133.858 89.916) (size 0.7112) (drill 0.4826) (layers "F.Cu" "B.Cu") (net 19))
 (segment (start 133.858 89.916) (end 133.858 108.204) (width 0.381) (layer "B.Cu") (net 19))
 (segment (start 143.002 110.998) (end 143.51 110.998) (width 0.381) (layer "F.Cu") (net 20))
 (segment (start 142.748 110.998) (end 143.002 110.998) (width 0.381) (layer "F.Cu") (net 20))
 (segment (start 123.66145 87.122) (end 132.334 87.122) (width 0.381) (layer "F.Cu") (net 20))
 (segment (start 132.334 110.998) (end 142.748 110.998) (width 0.381) (layer "F.Cu") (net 20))
 (segment (start 149.606 106.426) (end 150.114 105.918) (width 0.381) (layer "F.Cu") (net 20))
 (segment (start 148.082 106.426) (end 149.606 106.426) (width 0.381) (layer "F.Cu") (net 20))
 (segment (start 150.114 105.918) (end 150.114 104.14) (width 0.381) (layer "F.Cu") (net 20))
 (segment (start 147.828 106.68) (end 148.082 106.426) (width 0.381) (layer "F.Cu") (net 20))
 (segment (start 143.51 110.998) (end 147.828 106.68) (width 0.381) (layer "F.Cu") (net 20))
 (segment (start 121.58345 89.2) (end 123.66145 87.122) (width 0.381) (layer "F.Cu") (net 20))
 (via (at 132.334 87.122) (size 0.7112) (drill 0.4826) (layers "F.Cu" "B.Cu") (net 20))
 (via (at 132.334 110.998) (size 0.7112) (drill 0.4826) (layers "F.Cu" "B.Cu") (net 20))
 (segment (start 132.334 87.122) (end 132.334 110.998) (width 0.381) (layer "B.Cu") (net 20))
 (segment (start 121.58345 101.9) (end 118.03748 98.35403) (width 0.381) (layer "F.Cu") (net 10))
 (segment (start 152.4 88.646) (end 152.4 97.282) (width 0.381) (layer "F.Cu") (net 10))
 (segment (start 152.4 97.282) (end 151.892 97.79) (width 0.381) (layer "F.Cu") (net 10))
 (segment (start 119.888 85.09) (end 132.842 85.09) (width 0.381) (layer "F.Cu") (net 10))
 (segment (start 132.842 85.09) (end 134.62 86.868) (width 0.381) (layer "F.Cu") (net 10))
 (segment (start 118.03748 86.94052) (end 119.888 85.09) (width 0.381) (layer "F.Cu") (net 10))
 (segment (start 151.638 98.044) (end 150.114 98.044) (width 0.381) (layer "F.Cu") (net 10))
 (segment (start 118.03748 98.35403) (end 118.03748 86.94052) (width 0.381) (layer "F.Cu") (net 10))
 (segment (start 151.892 97.79) (end 151.638 98.044) (width 0.381) (layer "F.Cu") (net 10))
 (via (at 152.4 88.646) (size 0.7112) (drill 0.4826) (layers "F.Cu" "B.Cu") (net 10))
 (via (at 134.62 86.868) (size 0.7112) (drill 0.4826) (layers "F.Cu" "B.Cu") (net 10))
 (segment (start 150.622 86.868) (end 152.4 88.646) (width 0.381) (layer "B.Cu") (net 10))
 (segment (start 134.62 86.868) (end 150.622 86.868) (width 0.381) (layer "B.Cu") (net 10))
 (segment (start 153.67 98.044) (end 152.4 99.314) (width 0.381) (layer "F.Cu") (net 12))
 (segment (start 153.67 88.138) (end 153.67 98.044) (width 0.381) (layer "F.Cu") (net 12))
 (segment (start 152.4 99.314) (end 150.114 99.314) (width 0.381) (layer "F.Cu") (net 12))
 (via (at 153.67 88.138) (size 0.7112) (drill 0.4826) (layers "F.Cu" "B.Cu") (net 12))
 (segment (start 122.694261 84.836) (end 150.368 84.836) (width 0.381) (layer "B.Cu") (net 12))
 (segment (start 118.47296 96.24951) (end 118.47296 89.057301) (width 0.381) (layer "B.Cu") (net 12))
 (segment (start 121.58345 99.36) (end 118.47296 96.24951) (width 0.381) (layer "B.Cu") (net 12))
 (segment (start 118.47296 89.057301) (end 122.694261 84.836) (width 0.381) (layer "B.Cu") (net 12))
 (segment (start 150.368 84.836) (end 153.67 88.138) (width 0.381) (layer "B.Cu") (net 12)))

